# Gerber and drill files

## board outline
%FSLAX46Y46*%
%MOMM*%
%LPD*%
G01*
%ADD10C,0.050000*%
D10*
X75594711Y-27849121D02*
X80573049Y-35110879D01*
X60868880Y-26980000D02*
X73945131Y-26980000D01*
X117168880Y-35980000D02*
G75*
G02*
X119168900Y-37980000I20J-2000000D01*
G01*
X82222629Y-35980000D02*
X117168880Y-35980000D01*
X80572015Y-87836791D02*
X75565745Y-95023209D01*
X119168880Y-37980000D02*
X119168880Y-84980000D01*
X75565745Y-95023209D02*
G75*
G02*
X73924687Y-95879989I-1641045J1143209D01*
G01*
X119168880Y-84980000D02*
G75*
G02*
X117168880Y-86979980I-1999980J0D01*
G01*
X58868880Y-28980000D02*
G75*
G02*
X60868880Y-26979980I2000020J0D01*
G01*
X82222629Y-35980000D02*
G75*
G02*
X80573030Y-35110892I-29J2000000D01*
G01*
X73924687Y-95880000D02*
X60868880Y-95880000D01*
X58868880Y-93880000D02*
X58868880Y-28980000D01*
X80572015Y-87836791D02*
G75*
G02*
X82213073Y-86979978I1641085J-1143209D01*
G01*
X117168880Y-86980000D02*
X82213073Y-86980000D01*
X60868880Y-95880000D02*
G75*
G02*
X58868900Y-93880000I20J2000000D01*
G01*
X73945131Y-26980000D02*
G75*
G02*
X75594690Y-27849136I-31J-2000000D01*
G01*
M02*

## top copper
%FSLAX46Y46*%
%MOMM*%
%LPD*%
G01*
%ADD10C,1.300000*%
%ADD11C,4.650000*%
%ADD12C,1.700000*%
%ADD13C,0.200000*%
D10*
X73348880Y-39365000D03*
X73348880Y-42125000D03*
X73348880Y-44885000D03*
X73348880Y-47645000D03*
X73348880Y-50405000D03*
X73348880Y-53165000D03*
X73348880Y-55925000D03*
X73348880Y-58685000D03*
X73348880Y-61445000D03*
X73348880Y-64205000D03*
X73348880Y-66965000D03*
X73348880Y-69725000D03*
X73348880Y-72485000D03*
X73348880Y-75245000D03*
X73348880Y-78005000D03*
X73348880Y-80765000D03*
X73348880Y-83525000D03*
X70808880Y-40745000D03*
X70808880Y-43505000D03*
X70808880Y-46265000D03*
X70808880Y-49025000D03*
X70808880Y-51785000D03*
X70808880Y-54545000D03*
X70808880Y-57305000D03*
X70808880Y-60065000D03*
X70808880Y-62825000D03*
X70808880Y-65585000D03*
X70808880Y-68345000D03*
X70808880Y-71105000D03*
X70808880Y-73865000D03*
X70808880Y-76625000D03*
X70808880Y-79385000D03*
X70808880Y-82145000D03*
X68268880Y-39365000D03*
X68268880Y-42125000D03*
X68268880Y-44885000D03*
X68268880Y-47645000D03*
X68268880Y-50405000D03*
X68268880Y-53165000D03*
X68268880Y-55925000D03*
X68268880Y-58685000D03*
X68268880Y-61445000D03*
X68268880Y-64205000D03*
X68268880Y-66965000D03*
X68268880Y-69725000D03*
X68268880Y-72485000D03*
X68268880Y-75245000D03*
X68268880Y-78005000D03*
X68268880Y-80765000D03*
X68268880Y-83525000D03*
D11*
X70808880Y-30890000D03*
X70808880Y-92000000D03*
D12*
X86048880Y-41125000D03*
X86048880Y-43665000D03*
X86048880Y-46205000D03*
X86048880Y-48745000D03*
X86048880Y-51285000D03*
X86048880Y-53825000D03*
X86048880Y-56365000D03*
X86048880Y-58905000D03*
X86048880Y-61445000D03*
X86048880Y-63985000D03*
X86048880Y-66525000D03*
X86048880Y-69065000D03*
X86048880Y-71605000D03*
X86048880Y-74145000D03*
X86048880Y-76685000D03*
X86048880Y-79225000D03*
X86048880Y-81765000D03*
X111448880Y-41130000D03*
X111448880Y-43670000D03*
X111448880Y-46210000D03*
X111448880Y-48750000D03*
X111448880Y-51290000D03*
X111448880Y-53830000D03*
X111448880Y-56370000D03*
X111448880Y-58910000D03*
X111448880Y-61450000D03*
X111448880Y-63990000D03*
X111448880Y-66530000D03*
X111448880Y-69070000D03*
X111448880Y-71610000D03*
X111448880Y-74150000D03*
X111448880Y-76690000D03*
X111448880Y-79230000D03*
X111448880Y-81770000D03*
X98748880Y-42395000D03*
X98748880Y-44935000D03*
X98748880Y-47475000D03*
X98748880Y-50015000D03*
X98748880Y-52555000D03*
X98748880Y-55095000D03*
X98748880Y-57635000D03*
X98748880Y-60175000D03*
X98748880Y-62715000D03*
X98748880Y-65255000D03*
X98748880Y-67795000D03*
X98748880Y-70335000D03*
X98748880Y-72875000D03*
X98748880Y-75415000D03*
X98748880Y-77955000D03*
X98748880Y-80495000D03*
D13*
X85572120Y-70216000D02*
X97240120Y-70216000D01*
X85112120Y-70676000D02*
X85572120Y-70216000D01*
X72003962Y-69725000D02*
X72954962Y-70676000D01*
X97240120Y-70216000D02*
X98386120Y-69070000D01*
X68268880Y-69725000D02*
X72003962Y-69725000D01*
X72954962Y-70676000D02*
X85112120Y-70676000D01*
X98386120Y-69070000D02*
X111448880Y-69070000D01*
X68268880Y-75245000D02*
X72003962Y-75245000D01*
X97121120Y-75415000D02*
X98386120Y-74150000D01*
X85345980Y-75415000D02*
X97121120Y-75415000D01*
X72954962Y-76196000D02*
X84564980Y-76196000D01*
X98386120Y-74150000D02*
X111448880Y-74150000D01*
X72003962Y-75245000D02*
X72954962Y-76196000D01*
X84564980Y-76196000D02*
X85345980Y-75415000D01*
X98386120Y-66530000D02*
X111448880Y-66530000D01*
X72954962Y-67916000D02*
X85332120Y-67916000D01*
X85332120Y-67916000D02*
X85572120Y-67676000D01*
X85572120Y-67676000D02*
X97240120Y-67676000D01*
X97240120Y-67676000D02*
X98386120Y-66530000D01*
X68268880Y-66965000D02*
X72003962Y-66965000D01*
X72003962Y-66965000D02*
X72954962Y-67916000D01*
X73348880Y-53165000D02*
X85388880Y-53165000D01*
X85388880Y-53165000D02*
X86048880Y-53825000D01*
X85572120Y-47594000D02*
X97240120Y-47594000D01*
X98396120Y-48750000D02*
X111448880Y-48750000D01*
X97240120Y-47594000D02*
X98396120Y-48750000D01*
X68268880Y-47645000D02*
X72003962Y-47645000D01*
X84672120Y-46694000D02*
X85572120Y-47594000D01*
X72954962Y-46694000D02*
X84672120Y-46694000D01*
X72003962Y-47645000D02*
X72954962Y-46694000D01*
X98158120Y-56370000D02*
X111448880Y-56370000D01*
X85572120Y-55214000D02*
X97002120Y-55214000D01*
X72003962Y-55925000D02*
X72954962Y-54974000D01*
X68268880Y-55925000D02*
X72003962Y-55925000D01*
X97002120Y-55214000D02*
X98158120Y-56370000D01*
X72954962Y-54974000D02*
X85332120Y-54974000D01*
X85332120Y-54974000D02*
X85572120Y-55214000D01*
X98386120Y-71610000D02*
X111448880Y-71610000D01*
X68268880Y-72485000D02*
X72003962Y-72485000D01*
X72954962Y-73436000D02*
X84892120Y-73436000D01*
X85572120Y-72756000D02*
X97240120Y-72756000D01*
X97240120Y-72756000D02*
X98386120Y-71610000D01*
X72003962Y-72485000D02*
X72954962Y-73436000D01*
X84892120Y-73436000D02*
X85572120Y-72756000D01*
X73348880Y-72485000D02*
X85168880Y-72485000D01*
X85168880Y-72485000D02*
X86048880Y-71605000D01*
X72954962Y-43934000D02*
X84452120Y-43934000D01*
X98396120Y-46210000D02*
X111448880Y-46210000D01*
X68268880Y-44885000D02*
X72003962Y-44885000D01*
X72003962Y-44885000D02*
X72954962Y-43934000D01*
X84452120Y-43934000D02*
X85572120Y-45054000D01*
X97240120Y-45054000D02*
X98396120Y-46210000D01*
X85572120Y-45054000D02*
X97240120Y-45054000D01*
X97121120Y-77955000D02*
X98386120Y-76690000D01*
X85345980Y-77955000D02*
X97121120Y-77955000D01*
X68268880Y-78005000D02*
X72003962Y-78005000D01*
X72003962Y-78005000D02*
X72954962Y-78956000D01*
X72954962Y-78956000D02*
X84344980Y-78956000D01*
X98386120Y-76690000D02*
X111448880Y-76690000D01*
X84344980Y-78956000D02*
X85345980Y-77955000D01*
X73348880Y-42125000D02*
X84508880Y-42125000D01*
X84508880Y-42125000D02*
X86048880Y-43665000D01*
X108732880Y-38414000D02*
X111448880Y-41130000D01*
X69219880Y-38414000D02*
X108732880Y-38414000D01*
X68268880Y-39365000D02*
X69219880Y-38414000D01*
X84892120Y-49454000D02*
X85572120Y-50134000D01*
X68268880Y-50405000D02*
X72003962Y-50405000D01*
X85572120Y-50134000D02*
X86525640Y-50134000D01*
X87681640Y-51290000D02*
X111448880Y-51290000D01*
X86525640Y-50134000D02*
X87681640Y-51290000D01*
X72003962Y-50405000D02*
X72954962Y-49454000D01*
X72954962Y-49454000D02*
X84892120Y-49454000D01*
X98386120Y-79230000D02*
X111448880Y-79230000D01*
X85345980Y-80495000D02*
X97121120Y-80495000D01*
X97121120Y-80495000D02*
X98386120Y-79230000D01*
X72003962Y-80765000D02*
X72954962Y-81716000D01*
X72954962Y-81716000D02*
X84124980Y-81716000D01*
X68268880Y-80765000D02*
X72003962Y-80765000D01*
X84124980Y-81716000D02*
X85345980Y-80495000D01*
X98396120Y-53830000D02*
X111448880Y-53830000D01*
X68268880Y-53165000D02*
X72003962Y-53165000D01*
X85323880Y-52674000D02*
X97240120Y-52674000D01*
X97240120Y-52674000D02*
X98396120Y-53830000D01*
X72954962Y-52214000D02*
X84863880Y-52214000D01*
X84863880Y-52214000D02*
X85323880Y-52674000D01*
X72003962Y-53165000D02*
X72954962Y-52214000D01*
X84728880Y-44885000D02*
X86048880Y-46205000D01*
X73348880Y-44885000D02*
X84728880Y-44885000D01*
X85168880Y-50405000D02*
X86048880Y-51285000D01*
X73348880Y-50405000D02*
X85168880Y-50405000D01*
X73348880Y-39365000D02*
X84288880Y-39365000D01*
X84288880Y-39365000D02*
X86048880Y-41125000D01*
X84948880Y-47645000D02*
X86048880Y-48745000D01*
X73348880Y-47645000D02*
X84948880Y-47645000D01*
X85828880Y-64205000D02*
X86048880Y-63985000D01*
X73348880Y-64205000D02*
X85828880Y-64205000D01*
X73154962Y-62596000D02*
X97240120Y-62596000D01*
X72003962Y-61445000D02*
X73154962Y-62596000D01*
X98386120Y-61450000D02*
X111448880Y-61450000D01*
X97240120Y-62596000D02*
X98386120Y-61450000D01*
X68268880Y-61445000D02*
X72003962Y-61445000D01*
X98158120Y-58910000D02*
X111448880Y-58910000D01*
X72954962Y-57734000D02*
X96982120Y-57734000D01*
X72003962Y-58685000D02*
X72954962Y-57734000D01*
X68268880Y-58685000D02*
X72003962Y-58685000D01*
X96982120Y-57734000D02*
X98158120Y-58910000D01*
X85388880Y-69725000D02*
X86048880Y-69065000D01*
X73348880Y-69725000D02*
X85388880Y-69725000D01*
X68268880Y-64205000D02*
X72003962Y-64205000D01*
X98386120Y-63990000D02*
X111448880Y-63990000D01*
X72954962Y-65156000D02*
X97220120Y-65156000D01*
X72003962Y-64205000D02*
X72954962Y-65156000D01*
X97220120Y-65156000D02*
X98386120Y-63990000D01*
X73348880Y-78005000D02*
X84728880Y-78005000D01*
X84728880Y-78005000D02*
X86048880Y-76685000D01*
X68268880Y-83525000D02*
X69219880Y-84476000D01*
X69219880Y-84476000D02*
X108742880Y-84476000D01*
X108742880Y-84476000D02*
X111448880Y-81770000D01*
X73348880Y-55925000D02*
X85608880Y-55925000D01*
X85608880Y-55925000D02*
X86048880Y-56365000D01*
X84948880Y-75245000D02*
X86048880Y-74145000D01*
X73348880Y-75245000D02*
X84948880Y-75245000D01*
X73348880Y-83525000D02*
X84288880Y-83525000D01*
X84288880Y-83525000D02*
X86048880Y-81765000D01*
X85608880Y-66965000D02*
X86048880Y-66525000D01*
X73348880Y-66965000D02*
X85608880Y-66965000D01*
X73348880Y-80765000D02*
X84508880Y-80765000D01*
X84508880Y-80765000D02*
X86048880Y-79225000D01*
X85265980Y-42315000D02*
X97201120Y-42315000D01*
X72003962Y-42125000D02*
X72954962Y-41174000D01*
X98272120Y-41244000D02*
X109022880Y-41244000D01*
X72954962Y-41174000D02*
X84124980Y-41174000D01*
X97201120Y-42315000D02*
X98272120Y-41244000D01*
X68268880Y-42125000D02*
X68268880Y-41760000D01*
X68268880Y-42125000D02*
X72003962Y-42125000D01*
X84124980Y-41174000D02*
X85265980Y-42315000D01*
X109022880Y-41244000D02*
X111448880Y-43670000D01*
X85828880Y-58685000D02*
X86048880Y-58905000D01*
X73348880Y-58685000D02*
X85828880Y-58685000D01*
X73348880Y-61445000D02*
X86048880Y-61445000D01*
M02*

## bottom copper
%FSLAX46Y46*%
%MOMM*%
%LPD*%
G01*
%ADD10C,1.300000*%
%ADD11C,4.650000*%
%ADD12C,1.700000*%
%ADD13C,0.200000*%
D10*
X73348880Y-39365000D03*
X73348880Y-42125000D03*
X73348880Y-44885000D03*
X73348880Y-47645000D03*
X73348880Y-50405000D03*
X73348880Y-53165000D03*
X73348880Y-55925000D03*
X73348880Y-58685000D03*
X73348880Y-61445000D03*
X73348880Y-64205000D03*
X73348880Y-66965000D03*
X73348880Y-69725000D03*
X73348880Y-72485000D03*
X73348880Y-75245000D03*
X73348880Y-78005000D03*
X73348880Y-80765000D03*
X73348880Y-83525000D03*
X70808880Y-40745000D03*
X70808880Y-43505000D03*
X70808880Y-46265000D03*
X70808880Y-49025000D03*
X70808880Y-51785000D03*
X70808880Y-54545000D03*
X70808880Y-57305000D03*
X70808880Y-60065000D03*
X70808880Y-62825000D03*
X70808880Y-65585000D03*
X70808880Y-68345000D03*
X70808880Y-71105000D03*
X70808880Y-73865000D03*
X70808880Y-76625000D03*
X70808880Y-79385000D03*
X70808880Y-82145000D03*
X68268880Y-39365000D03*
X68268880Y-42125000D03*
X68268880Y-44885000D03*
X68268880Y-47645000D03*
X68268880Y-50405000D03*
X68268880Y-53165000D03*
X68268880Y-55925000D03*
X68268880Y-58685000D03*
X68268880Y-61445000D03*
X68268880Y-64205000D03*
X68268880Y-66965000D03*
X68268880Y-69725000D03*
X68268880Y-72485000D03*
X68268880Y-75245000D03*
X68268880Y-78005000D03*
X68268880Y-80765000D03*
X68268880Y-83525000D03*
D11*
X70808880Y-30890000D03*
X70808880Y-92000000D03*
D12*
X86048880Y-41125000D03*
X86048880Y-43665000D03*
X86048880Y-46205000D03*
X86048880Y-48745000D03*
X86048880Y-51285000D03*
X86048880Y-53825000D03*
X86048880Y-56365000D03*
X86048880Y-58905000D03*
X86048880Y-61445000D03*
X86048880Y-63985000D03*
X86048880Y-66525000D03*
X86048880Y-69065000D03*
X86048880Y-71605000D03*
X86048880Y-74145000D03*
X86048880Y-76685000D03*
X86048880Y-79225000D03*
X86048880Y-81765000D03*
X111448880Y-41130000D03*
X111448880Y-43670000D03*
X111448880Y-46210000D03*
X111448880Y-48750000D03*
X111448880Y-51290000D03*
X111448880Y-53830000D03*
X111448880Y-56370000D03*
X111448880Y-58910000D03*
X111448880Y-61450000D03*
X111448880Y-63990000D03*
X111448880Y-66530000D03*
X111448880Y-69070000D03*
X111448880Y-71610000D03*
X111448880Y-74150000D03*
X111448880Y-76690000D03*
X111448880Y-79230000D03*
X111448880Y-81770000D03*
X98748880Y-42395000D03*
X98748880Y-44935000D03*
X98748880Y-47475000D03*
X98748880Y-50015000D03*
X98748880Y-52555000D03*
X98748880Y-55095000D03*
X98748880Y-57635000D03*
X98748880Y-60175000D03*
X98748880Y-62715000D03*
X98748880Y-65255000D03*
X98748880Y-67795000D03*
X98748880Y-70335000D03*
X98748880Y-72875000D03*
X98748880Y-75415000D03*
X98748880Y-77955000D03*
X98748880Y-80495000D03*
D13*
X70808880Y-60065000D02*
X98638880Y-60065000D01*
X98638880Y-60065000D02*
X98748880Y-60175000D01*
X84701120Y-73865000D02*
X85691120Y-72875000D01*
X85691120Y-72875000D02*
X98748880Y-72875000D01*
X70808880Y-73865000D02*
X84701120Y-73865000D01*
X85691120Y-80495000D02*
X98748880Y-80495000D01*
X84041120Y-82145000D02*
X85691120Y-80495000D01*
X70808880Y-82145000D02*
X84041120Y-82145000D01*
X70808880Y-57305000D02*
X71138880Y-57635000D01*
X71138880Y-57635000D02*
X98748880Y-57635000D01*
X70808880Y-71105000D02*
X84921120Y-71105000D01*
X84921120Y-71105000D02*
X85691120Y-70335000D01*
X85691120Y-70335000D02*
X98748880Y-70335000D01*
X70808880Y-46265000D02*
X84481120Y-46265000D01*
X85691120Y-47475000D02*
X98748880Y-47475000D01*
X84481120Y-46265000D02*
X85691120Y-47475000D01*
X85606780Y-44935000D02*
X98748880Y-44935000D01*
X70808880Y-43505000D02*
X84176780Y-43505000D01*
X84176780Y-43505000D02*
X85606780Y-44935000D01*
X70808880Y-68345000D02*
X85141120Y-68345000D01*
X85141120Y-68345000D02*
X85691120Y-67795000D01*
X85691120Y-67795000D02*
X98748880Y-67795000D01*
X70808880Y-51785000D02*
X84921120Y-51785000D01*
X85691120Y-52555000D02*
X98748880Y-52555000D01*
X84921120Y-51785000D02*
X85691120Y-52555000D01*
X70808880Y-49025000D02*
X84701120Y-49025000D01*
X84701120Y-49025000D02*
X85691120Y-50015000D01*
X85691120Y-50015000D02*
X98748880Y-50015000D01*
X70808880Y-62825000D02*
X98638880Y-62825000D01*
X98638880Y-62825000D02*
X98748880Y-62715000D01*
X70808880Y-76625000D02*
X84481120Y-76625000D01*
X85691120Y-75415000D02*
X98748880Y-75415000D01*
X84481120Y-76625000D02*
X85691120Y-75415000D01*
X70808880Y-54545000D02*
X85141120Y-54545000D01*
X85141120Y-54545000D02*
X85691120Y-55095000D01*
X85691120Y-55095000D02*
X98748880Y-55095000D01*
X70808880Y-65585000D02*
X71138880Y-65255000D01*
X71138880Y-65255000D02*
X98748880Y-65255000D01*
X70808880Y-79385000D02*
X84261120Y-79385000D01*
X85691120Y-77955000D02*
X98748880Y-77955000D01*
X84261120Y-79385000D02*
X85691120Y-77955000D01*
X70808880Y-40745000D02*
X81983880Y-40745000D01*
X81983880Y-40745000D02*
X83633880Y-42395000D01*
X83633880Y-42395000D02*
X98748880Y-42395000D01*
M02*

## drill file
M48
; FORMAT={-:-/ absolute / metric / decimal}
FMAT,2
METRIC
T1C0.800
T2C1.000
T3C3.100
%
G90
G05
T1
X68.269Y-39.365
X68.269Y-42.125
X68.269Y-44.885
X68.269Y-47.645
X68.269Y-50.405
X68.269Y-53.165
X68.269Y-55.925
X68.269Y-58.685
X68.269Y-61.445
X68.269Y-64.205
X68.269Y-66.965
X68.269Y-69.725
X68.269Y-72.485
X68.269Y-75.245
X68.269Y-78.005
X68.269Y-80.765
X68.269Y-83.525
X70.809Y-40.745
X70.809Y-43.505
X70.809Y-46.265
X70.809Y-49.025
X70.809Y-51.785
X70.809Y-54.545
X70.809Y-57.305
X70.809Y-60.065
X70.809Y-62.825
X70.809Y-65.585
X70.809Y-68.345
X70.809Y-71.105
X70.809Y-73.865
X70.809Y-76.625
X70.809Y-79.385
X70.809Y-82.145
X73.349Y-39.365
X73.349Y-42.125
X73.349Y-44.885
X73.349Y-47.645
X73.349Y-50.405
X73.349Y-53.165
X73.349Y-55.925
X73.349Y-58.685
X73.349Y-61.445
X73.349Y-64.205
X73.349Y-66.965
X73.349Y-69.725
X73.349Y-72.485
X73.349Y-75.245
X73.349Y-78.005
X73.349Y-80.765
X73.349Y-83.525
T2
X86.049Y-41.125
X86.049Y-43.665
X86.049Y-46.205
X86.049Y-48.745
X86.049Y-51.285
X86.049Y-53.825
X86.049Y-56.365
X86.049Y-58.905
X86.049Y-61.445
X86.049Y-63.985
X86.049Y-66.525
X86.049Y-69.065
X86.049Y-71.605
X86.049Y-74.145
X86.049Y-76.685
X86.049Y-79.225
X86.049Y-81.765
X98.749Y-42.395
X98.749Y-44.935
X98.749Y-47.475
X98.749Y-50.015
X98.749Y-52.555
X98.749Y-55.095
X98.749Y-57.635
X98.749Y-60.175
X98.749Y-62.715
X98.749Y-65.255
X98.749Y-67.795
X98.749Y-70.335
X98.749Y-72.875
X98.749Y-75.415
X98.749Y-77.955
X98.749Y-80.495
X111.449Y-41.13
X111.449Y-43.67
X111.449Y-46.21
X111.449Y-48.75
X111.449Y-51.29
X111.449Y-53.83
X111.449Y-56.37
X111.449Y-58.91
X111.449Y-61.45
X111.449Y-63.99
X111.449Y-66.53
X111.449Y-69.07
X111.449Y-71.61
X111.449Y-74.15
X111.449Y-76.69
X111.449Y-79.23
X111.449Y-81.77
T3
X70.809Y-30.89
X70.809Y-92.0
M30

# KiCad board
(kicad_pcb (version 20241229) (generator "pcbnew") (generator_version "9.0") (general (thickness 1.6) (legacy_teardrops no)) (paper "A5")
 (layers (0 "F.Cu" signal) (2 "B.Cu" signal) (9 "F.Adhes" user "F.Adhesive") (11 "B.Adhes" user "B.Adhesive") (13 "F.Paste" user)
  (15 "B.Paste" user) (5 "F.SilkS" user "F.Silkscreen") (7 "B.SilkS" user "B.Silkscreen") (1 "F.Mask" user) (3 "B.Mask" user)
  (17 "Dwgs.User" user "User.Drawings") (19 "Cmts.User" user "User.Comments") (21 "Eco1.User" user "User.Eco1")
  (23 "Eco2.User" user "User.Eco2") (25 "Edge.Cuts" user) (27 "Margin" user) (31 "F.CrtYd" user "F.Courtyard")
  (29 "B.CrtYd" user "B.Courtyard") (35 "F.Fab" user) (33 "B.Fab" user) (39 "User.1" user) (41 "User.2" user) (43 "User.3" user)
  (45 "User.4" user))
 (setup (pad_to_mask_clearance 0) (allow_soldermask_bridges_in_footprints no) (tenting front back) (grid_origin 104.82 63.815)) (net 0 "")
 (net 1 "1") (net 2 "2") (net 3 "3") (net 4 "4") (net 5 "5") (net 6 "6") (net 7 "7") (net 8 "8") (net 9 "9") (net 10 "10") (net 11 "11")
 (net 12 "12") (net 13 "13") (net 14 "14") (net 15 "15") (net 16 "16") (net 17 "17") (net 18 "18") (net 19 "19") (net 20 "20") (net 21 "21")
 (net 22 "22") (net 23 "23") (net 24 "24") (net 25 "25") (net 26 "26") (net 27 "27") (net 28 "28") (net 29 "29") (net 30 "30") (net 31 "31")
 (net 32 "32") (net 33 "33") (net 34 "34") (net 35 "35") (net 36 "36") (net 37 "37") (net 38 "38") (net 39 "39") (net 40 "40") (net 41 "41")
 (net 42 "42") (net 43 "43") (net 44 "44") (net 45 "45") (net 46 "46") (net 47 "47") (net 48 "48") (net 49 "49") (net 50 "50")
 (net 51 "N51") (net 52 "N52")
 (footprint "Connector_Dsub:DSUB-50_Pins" (layer "F.Cu") (at 73.34888 39.365 -90)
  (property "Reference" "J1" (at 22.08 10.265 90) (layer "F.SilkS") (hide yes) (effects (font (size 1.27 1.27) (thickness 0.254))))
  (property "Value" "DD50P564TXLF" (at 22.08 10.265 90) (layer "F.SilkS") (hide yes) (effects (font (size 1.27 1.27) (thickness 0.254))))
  (pad "1" thru_hole circle (at 0 0 270) (size 1.3 1.3) (drill 0.8) (layers "*.Cu" "*.Mask") (remove_unused_layers no) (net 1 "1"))
  (pad "2" thru_hole circle (at 2.76 0 270) (size 1.3 1.3) (drill 0.8) (layers "*.Cu" "*.Mask") (remove_unused_layers no) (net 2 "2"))
  (pad "3" thru_hole circle (at 5.52 0 270) (size 1.3 1.3) (drill 0.8) (layers "*.Cu" "*.Mask") (remove_unused_layers no) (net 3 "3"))
  (pad "4" thru_hole circle (at 8.28 0 270) (size 1.3 1.3) (drill 0.8) (layers "*.Cu" "*.Mask") (remove_unused_layers no) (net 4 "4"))
  (pad "5" thru_hole circle (at 11.04 0 270) (size 1.3 1.3) (drill 0.8) (layers "*.Cu" "*.Mask") (remove_unused_layers no) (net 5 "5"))
  (pad "6" thru_hole circle (at 13.8 0 270) (size 1.3 1.3) (drill 0.8) (layers "*.Cu" "*.Mask") (remove_unused_layers no) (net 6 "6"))
  (pad "7" thru_hole circle (at 16.56 0 270) (size 1.3 1.3) (drill 0.8) (layers "*.Cu" "*.Mask") (remove_unused_layers no) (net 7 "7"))
  (pad "8" thru_hole circle (at 19.32 0 270) (size 1.3 1.3) (drill 0.8) (layers "*.Cu" "*.Mask") (remove_unused_layers no) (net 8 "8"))
  (pad "9" thru_hole circle (at 22.08 0 270) (size 1.3 1.3) (drill 0.8) (layers "*.Cu" "*.Mask") (remove_unused_layers no) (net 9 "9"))
  (pad "10" thru_hole circle (at 24.84 0 270) (size 1.3 1.3) (drill 0.8) (layers "*.Cu" "*.Mask") (remove_unused_layers no) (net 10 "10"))
  (pad "11" thru_hole circle (at 27.6 0 270) (size 1.3 1.3) (drill 0.8) (layers "*.Cu" "*.Mask") (remove_unused_layers no) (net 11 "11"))
  (pad "12" thru_hole circle (at 30.36 0 270) (size 1.3 1.3) (drill 0.8) (layers "*.Cu" "*.Mask") (remove_unused_layers no) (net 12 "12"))
  (pad "13" thru_hole circle (at 33.12 0 270) (size 1.3 1.3) (drill 0.8) (layers "*.Cu" "*.Mask") (remove_unused_layers no) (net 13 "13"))
  (pad "14" thru_hole circle (at 35.88 0 270) (size 1.3 1.3) (drill 0.8) (layers "*.Cu" "*.Mask") (remove_unused_layers no) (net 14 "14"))
  (pad "15" thru_hole circle (at 38.64 0 270) (size 1.3 1.3) (drill 0.8) (layers "*.Cu" "*.Mask") (remove_unused_layers no) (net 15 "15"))
  (pad "16" thru_hole circle (at 41.4 0 270) (size 1.3 1.3) (drill 0.8) (layers "*.Cu" "*.Mask") (remove_unused_layers no) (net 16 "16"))
  (pad "17" thru_hole circle (at 44.16 0 270) (size 1.3 1.3) (drill 0.8) (layers "*.Cu" "*.Mask") (remove_unused_layers no) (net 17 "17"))
  (pad "18" thru_hole circle (at 1.38 2.54 270) (size 1.3 1.3) (drill 0.8) (layers "*.Cu" "*.Mask") (remove_unused_layers no) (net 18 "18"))
  (pad "19" thru_hole circle (at 4.14 2.54 270) (size 1.3 1.3) (drill 0.8) (layers "*.Cu" "*.Mask") (remove_unused_layers no) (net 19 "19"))
  (pad "20" thru_hole circle (at 6.9 2.54 270) (size 1.3 1.3) (drill 0.8) (layers "*.Cu" "*.Mask") (remove_unused_layers no) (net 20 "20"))
  (pad "21" thru_hole circle (at 9.66 2.54 270) (size 1.3 1.3) (drill 0.8) (layers "*.Cu" "*.Mask") (remove_unused_layers no) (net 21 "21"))
  (pad "22" thru_hole circle (at 12.42 2.54 270) (size 1.3 1.3) (drill 0.8) (layers "*.Cu" "*.Mask") (remove_unused_layers no) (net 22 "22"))
  (pad "23" thru_hole circle (at 15.18 2.54 270) (size 1.3 1.3) (drill 0.8) (layers "*.Cu" "*.Mask") (remove_unused_layers no) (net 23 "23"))
  (pad "24" thru_hole circle (at 17.94 2.54 270) (size 1.3 1.3) (drill 0.8) (layers "*.Cu" "*.Mask") (remove_unused_layers no) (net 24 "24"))
  (pad "25" thru_hole circle (at 20.7 2.54 270) (size 1.3 1.3) (drill 0.8) (layers "*.Cu" "*.Mask") (remove_unused_layers no) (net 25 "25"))
  (pad "26" thru_hole circle (at 23.46 2.54 270) (size 1.3 1.3) (drill 0.8) (layers "*.Cu" "*.Mask") (remove_unused_layers no) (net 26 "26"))
  (pad "27" thru_hole circle (at 26.22 2.54 270) (size 1.3 1.3) (drill 0.8) (layers "*.Cu" "*.Mask") (remove_unused_layers no) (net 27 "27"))
  (pad "28" thru_hole circle (at 28.98 2.54 270) (size 1.3 1.3) (drill 0.8) (layers "*.Cu" "*.Mask") (remove_unused_layers no) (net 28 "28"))
  (pad "29" thru_hole circle (at 31.74 2.54 270) (size 1.3 1.3) (drill 0.8) (layers "*.Cu" "*.Mask") (remove_unused_layers no) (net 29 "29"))
  (pad "30" thru_hole circle (at 34.5 2.54 270) (size 1.3 1.3) (drill 0.8) (layers "*.Cu" "*.Mask") (remove_unused_layers no) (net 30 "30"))
  (pad "31" thru_hole circle (at 37.26 2.54 270) (size 1.3 1.3) (drill 0.8) (layers "*.Cu" "*.Mask") (remove_unused_layers no) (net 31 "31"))
  (pad "32" thru_hole circle (at 40.02 2.54 270) (size 1.3 1.3) (drill 0.8) (layers "*.Cu" "*.Mask") (remove_unused_layers no) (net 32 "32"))
  (pad "33" thru_hole circle (at 42.78 2.54 270) (size 1.3 1.3) (drill 0.8) (layers "*.Cu" "*.Mask") (remove_unused_layers no) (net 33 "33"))
  (pad "34" thru_hole circle (at 0 5.08 270) (size 1.3 1.3) (drill 0.8) (layers "*.Cu" "*.Mask") (remove_unused_layers no) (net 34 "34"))
  (pad "35" thru_hole circle (at 2.76 5.08 270) (size 1.3 1.3) (drill 0.8) (layers "*.Cu" "*.Mask") (remove_unused_layers no) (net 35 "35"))
  (pad "36" thru_hole circle (at 5.52 5.08 270) (size 1.3 1.3) (drill 0.8) (layers "*.Cu" "*.Mask") (remove_unused_layers no) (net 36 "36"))
  (pad "37" thru_hole circle (at 8.28 5.08 270) (size 1.3 1.3) (drill 0.8) (layers "*.Cu" "*.Mask") (remove_unused_layers no) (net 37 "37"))
  (pad "38" thru_hole circle (at 11.04 5.08 270) (size 1.3 1.3) (drill 0.8) (layers "*.Cu" "*.Mask") (remove_unused_layers no) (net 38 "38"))
  (pad "39" thru_hole circle (at 13.8 5.08 270) (size 1.3 1.3) (drill 0.8) (layers "*.Cu" "*.Mask") (remove_unused_layers no) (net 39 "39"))
  (pad "40" thru_hole circle (at 16.56 5.08 270) (size 1.3 1.3) (drill 0.8) (layers "*.Cu" "*.Mask") (remove_unused_layers no) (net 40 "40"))
  (pad "41" thru_hole circle (at 19.32 5.08 270) (size 1.3 1.3) (drill 0.8) (layers "*.Cu" "*.Mask") (remove_unused_layers no) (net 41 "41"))
  (pad "42" thru_hole circle (at 22.08 5.08 270) (size 1.3 1.3) (drill 0.8) (layers "*.Cu" "*.Mask") (remove_unused_layers no) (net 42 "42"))
  (pad "43" thru_hole circle (at 24.84 5.08 270) (size 1.3 1.3) (drill 0.8) (layers "*.Cu" "*.Mask") (remove_unused_layers no) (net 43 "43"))
  (pad "44" thru_hole circle (at 27.6 5.08 270) (size 1.3 1.3) (drill 0.8) (layers "*.Cu" "*.Mask") (remove_unused_layers no) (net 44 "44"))
  (pad "45" thru_hole circle (at 30.36 5.08 270) (size 1.3 1.3) (drill 0.8) (layers "*.Cu" "*.Mask") (remove_unused_layers no) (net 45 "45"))
  (pad "46" thru_hole circle (at 33.12 5.08 270) (size 1.3 1.3) (drill 0.8) (layers "*.Cu" "*.Mask") (remove_unused_layers no) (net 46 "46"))
  (pad "47" thru_hole circle (at 35.88 5.08 270) (size 1.3 1.3) (drill 0.8) (layers "*.Cu" "*.Mask") (remove_unused_layers no) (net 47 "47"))
  (pad "48" thru_hole circle (at 38.64 5.08 270) (size 1.3 1.3) (drill 0.8) (layers "*.Cu" "*.Mask") (remove_unused_layers no) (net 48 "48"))
  (pad "49" thru_hole circle (at 41.4 5.08 270) (size 1.3 1.3) (drill 0.8) (layers "*.Cu" "*.Mask") (remove_unused_layers no) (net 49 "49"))
  (pad "50" thru_hole circle (at 44.16 5.08 270) (size 1.3 1.3) (drill 0.8) (layers "*.Cu" "*.Mask") (remove_unused_layers no) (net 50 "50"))
  (pad "MH1" thru_hole circle (at -8.475 2.54 270) (size 4.65 4.65) (drill 3.1) (layers "*.Cu" "*.Mask") (remove_unused_layers no)
   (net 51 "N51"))
  (pad "MH2" thru_hole circle (at 52.635 2.54 270) (size 4.65 4.65) (drill 3.1) (layers "*.Cu" "*.Mask") (remove_unused_layers no)
   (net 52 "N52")))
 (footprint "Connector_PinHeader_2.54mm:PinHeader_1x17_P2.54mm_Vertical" (layer "F.Cu") (at 86.04888 41.125)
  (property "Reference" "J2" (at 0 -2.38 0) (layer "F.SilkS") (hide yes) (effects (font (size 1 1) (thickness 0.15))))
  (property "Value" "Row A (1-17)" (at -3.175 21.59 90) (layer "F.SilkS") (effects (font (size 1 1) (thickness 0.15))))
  (pad "1" thru_hole circle (at 0 0) (size 1.7 1.7) (drill 1) (layers "*.Cu" "*.Mask") (remove_unused_layers no) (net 1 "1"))
  (pad "2" thru_hole circle (at 0 2.54) (size 1.7 1.7) (drill 1) (layers "*.Cu" "*.Mask") (remove_unused_layers no) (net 2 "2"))
  (pad "3" thru_hole circle (at 0 5.08) (size 1.7 1.7) (drill 1) (layers "*.Cu" "*.Mask") (remove_unused_layers no) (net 3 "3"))
  (pad "4" thru_hole circle (at 0 7.62) (size 1.7 1.7) (drill 1) (layers "*.Cu" "*.Mask") (remove_unused_layers no) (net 4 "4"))
  (pad "5" thru_hole circle (at 0 10.16) (size 1.7 1.7) (drill 1) (layers "*.Cu" "*.Mask") (remove_unused_layers no) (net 5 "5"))
  (pad "6" thru_hole circle (at 0 12.7) (size 1.7 1.7) (drill 1) (layers "*.Cu" "*.Mask") (remove_unused_layers no) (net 6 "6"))
  (pad "7" thru_hole circle (at 0 15.24) (size 1.7 1.7) (drill 1) (layers "*.Cu" "*.Mask") (remove_unused_layers no) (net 7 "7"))
  (pad "8" thru_hole circle (at 0 17.78) (size 1.7 1.7) (drill 1) (layers "*.Cu" "*.Mask") (remove_unused_layers no) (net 8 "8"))
  (pad "9" thru_hole circle (at 0 20.32) (size 1.7 1.7) (drill 1) (layers "*.Cu" "*.Mask") (remove_unused_layers no) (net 9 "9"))
  (pad "10" thru_hole circle (at 0 22.86) (size 1.7 1.7) (drill 1) (layers "*.Cu" "*.Mask") (remove_unused_layers no) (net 10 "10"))
  (pad "11" thru_hole circle (at 0 25.4) (size 1.7 1.7) (drill 1) (layers "*.Cu" "*.Mask") (remove_unused_layers no) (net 11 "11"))
  (pad "12" thru_hole circle (at 0 27.94) (size 1.7 1.7) (drill 1) (layers "*.Cu" "*.Mask") (remove_unused_layers no) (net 12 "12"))
  (pad "13" thru_hole circle (at 0 30.48) (size 1.7 1.7) (drill 1) (layers "*.Cu" "*.Mask") (remove_unused_layers no) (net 13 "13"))
  (pad "14" thru_hole circle (at 0 33.02) (size 1.7 1.7) (drill 1) (layers "*.Cu" "*.Mask") (remove_unused_layers no) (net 14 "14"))
  (pad "15" thru_hole circle (at 0 35.56) (size 1.7 1.7) (drill 1) (layers "*.Cu" "*.Mask") (remove_unused_layers no) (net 15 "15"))
  (pad "16" thru_hole circle (at 0 38.1) (size 1.7 1.7) (drill 1) (layers "*.Cu" "*.Mask") (remove_unused_layers no) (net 16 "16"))
  (pad "17" thru_hole circle (at 0 40.64) (size 1.7 1.7) (drill 1) (layers "*.Cu" "*.Mask") (remove_unused_layers no) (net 17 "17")))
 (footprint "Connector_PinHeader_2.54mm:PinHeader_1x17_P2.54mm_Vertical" (layer "F.Cu") (at 111.44888 41.13)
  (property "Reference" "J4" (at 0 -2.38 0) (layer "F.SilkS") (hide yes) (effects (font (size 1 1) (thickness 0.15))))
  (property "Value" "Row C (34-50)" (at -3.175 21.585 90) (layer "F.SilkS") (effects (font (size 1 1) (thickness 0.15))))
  (pad "1" thru_hole circle (at 0 0) (size 1.7 1.7) (drill 1) (layers "*.Cu" "*.Mask") (remove_unused_layers no) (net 34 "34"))
  (pad "2" thru_hole circle (at 0 2.54) (size 1.7 1.7) (drill 1) (layers "*.Cu" "*.Mask") (remove_unused_layers no) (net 35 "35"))
  (pad "3" thru_hole circle (at 0 5.08) (size 1.7 1.7) (drill 1) (layers "*.Cu" "*.Mask") (remove_unused_layers no) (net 36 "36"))
  (pad "4" thru_hole circle (at 0 7.62) (size 1.7 1.7) (drill 1) (layers "*.Cu" "*.Mask") (remove_unused_layers no) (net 37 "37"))
  (pad "5" thru_hole circle (at 0 10.16) (size 1.7 1.7) (drill 1) (layers "*.Cu" "*.Mask") (remove_unused_layers no) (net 38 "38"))
  (pad "6" thru_hole circle (at 0 12.7) (size 1.7 1.7) (drill 1) (layers "*.Cu" "*.Mask") (remove_unused_layers no) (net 39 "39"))
  (pad "7" thru_hole circle (at 0 15.24) (size 1.7 1.7) (drill 1) (layers "*.Cu" "*.Mask") (remove_unused_layers no) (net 40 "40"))
  (pad "8" thru_hole circle (at 0 17.78) (size 1.7 1.7) (drill 1) (layers "*.Cu" "*.Mask") (remove_unused_layers no) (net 41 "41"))
  (pad "9" thru_hole circle (at 0 20.32) (size 1.7 1.7) (drill 1) (layers "*.Cu" "*.Mask") (remove_unused_layers no) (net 42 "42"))
  (pad "10" thru_hole circle (at 0 22.86) (size 1.7 1.7) (drill 1) (layers "*.Cu" "*.Mask") (remove_unused_layers no) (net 43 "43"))
  (pad "11" thru_hole circle (at 0 25.4) (size 1.7 1.7) (drill 1) (layers "*.Cu" "*.Mask") (remove_unused_layers no) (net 44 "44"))
  (pad "12" thru_hole circle (at 0 27.94) (size 1.7 1.7) (drill 1) (layers "*.Cu" "*.Mask") (remove_unused_layers no) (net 45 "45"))
  (pad "13" thru_hole circle (at 0 30.48) (size 1.7 1.7) (drill 1) (layers "*.Cu" "*.Mask") (remove_unused_layers no) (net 46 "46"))
  (pad "14" thru_hole circle (at 0 33.02) (size 1.7 1.7) (drill 1) (layers "*.Cu" "*.Mask") (remove_unused_layers no) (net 47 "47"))
  (pad "15" thru_hole circle (at 0 35.56) (size 1.7 1.7) (drill 1) (layers "*.Cu" "*.Mask") (remove_unused_layers no) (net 48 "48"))
  (pad "16" thru_hole circle (at 0 38.1) (size 1.7 1.7) (drill 1) (layers "*.Cu" "*.Mask") (remove_unused_layers no) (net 49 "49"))
  (pad "17" thru_hole circle (at 0 40.64) (size 1.7 1.7) (drill 1) (layers "*.Cu" "*.Mask") (remove_unused_layers no) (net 50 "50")))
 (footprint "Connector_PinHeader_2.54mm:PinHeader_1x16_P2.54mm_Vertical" (layer "F.Cu") (at 98.74888 42.395)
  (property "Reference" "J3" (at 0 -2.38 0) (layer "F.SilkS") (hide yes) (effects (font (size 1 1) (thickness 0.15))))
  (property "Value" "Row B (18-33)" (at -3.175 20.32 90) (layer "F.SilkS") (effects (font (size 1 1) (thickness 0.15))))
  (pad "1" thru_hole circle (at 0 0) (size 1.7 1.7) (drill 1) (layers "*.Cu" "*.Mask") (remove_unused_layers no) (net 18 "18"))
  (pad "2" thru_hole circle (at 0 2.54) (size 1.7 1.7) (drill 1) (layers "*.Cu" "*.Mask") (remove_unused_layers no) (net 19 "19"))
  (pad "3" thru_hole circle (at 0 5.08) (size 1.7 1.7) (drill 1) (layers "*.Cu" "*.Mask") (remove_unused_layers no) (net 20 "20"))
  (pad "4" thru_hole circle (at 0 7.62) (size 1.7 1.7) (drill 1) (layers "*.Cu" "*.Mask") (remove_unused_layers no) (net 21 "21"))
  (pad "5" thru_hole circle (at 0 10.16) (size 1.7 1.7) (drill 1) (layers "*.Cu" "*.Mask") (remove_unused_layers no) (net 22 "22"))
  (pad "6" thru_hole circle (at 0 12.7) (size 1.7 1.7) (drill 1) (layers "*.Cu" "*.Mask") (remove_unused_layers no) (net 23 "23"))
  (pad "7" thru_hole circle (at 0 15.24) (size 1.7 1.7) (drill 1) (layers "*.Cu" "*.Mask") (remove_unused_layers no) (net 24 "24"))
  (pad "8" thru_hole circle (at 0 17.78) (size 1.7 1.7) (drill 1) (layers "*.Cu" "*.Mask") (remove_unused_layers no) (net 25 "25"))
  (pad "9" thru_hole circle (at 0 20.32) (size 1.7 1.7) (drill 1) (layers "*.Cu" "*.Mask") (remove_unused_layers no) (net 26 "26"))
  (pad "10" thru_hole circle (at 0 22.86) (size 1.7 1.7) (drill 1) (layers "*.Cu" "*.Mask") (remove_unused_layers no) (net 27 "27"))
  (pad "11" thru_hole circle (at 0 25.4) (size 1.7 1.7) (drill 1) (layers "*.Cu" "*.Mask") (remove_unused_layers no) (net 28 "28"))
  (pad "12" thru_hole circle (at 0 27.94) (size 1.7 1.7) (drill 1) (layers "*.Cu" "*.Mask") (remove_unused_layers no) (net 29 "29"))
  (pad "13" thru_hole circle (at 0 30.48) (size 1.7 1.7) (drill 1) (layers "*.Cu" "*.Mask") (remove_unused_layers no) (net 30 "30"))
  (pad "14" thru_hole circle (at 0 33.02) (size 1.7 1.7) (drill 1) (layers "*.Cu" "*.Mask") (remove_unused_layers no) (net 31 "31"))
  (pad "15" thru_hole circle (at 0 35.56) (size 1.7 1.7) (drill 1) (layers "*.Cu" "*.Mask") (remove_unused_layers no) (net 32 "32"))
  (pad "16" thru_hole circle (at 0 38.1) (size 1.7 1.7) (drill 1) (layers "*.Cu" "*.Mask") (remove_unused_layers no) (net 33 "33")))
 (gr_line (start 75.594711 27.849121) (end 80.573049 35.110879) (stroke (width 0.05) (type default)) (layer "Edge.Cuts"))
 (gr_line (start 60.86888 26.98) (end 73.945131 26.98) (stroke (width 0.05) (type default)) (layer "Edge.Cuts"))
 (gr_arc (start 117.16888 35.98) (mid 118.583094 36.565786) (end 119.16888 37.98) (stroke (width 0.05) (type default)) (layer "Edge.Cuts"))
 (gr_line (start 82.222629 35.98) (end 117.16888 35.98) (stroke (width 0.05) (type default)) (layer "Edge.Cuts"))
 (gr_line (start 80.572015 87.836791) (end 75.565745 95.023209) (stroke (width 0.05) (type default)) (layer "Edge.Cuts"))
 (gr_line (start 119.16888 37.98) (end 119.16888 84.98) (stroke (width 0.05) (type default)) (layer "Edge.Cuts"))
 (gr_arc (start 75.565745 95.023209) (mid 74.850317 95.652909) (end 73.924687 95.88) (stroke (width 0.05) (type default))
  (layer "Edge.Cuts"))
 (gr_arc (start 119.16888 84.98) (mid 118.583094 86.394214) (end 117.16888 86.98) (stroke (width 0.05) (type default)) (layer "Edge.Cuts"))
 (gr_arc (start 58.86888 28.98) (mid 59.454666 27.565786) (end 60.86888 26.98) (stroke (width 0.05) (type default)) (layer "Edge.Cuts"))
 (gr_arc (start 82.222629 35.98) (mid 81.290362 35.749429) (end 80.573049 35.110879) (stroke (width 0.05) (type default))
  (layer "Edge.Cuts"))
 (gr_line (start 73.924687 95.88) (end 60.86888 95.88) (stroke (width 0.05) (type default)) (layer "Edge.Cuts"))
 (gr_line (start 58.86888 93.88) (end 58.86888 28.98) (stroke (width 0.05) (type default)) (layer "Edge.Cuts"))
 (gr_arc (start 80.572015 87.836791) (mid 81.287443 87.207091) (end 82.213073 86.98) (stroke (width 0.05) (type default))
  (layer "Edge.Cuts"))
 (gr_line (start 117.16888 86.98) (end 82.213073 86.98) (stroke (width 0.05) (type default)) (layer "Edge.Cuts"))
 (gr_arc (start 60.86888 95.88) (mid 59.454666 95.294214) (end 58.86888 93.88) (stroke (width 0.05) (type default)) (layer "Edge.Cuts"))
 (gr_arc (start 73.945131 26.98) (mid 74.877398 27.210571) (end 75.594711 27.849121) (stroke (width 0.05) (type default))
  (layer "Edge.Cuts"))
 (segment (start 85.57212 70.216) (end 97.24012 70.216) (width 0.2) (layer "F.Cu") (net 45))
 (segment (start 85.11212 70.676) (end 85.57212 70.216) (width 0.2) (layer "F.Cu") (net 45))
 (segment (start 72.003962 69.725) (end 72.954962 70.676) (width 0.2) (layer "F.Cu") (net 45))
 (segment (start 97.24012 70.216) (end 98.38612 69.07) (width 0.2) (layer "F.Cu") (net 45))
 (segment (start 68.26888 69.725) (end 72.003962 69.725) (width 0.2) (layer "F.Cu") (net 45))
 (segment (start 72.954962 70.676) (end 85.11212 70.676) (width 0.2) (layer "F.Cu") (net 45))
 (segment (start 98.38612 69.07) (end 111.44888 69.07) (width 0.2) (layer "F.Cu") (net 45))
 (segment (start 68.26888 75.245) (end 72.003962 75.245) (width 0.2) (layer "F.Cu") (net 47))
 (segment (start 97.12112 75.415) (end 98.38612 74.15) (width 0.2) (layer "F.Cu") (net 47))
 (segment (start 85.34598 75.415) (end 97.12112 75.415) (width 0.2) (layer "F.Cu") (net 47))
 (segment (start 72.954962 76.196) (end 84.56498 76.196) (width 0.2) (layer "F.Cu") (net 47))
 (segment (start 98.38612 74.15) (end 111.44888 74.15) (width 0.2) (layer "F.Cu") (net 47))
 (segment (start 72.003962 75.245) (end 72.954962 76.196) (width 0.2) (layer "F.Cu") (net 47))
 (segment (start 84.56498 76.196) (end 85.34598 75.415) (width 0.2) (layer "F.Cu") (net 47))
 (segment (start 70.80888 60.065) (end 98.63888 60.065) (width 0.2) (layer "B.Cu") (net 25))
 (segment (start 98.63888 60.065) (end 98.74888 60.175) (width 0.2) (layer "B.Cu") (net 25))
 (segment (start 98.38612 66.53) (end 111.44888 66.53) (width 0.2) (layer "F.Cu") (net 44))
 (segment (start 72.954962 67.916) (end 85.33212 67.916) (width 0.2) (layer "F.Cu") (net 44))
 (segment (start 85.33212 67.916) (end 85.57212 67.676) (width 0.2) (layer "F.Cu") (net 44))
 (segment (start 85.57212 67.676) (end 97.24012 67.676) (width 0.2) (layer "F.Cu") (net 44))
 (segment (start 97.24012 67.676) (end 98.38612 66.53) (width 0.2) (layer "F.Cu") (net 44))
 (segment (start 68.26888 66.965) (end 72.003962 66.965) (width 0.2) (layer "F.Cu") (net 44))
 (segment (start 72.003962 66.965) (end 72.954962 67.916) (width 0.2) (layer "F.Cu") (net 44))
 (segment (start 73.34888 53.165) (end 85.38888 53.165) (width 0.2) (layer "F.Cu") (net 6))
 (segment (start 85.38888 53.165) (end 86.04888 53.825) (width 0.2) (layer "F.Cu") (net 6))
 (segment (start 85.57212 47.594) (end 97.24012 47.594) (width 0.2) (layer "F.Cu") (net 37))
 (segment (start 98.39612 48.75) (end 111.44888 48.75) (width 0.2) (layer "F.Cu") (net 37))
 (segment (start 97.24012 47.594) (end 98.39612 48.75) (width 0.2) (layer "F.Cu") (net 37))
 (segment (start 68.26888 47.645) (end 72.003962 47.645) (width 0.2) (layer "F.Cu") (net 37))
 (segment (start 84.67212 46.694) (end 85.57212 47.594) (width 0.2) (layer "F.Cu") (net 37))
 (segment (start 72.954962 46.694) (end 84.67212 46.694) (width 0.2) (layer "F.Cu") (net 37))
 (segment (start 72.003962 47.645) (end 72.954962 46.694) (width 0.2) (layer "F.Cu") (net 37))
 (segment (start 84.70112 73.865) (end 85.69112 72.875) (width 0.2) (layer "B.Cu") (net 30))
 (segment (start 85.69112 72.875) (end 98.74888 72.875) (width 0.2) (layer "B.Cu") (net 30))
 (segment (start 70.80888 73.865) (end 84.70112 73.865) (width 0.2) (layer "B.Cu") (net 30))
 (segment (start 85.69112 80.495) (end 98.74888 80.495) (width 0.2) (layer "B.Cu") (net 33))
 (segment (start 84.04112 82.145) (end 85.69112 80.495) (width 0.2) (layer "B.Cu") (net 33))
 (segment (start 70.80888 82.145) (end 84.04112 82.145) (width 0.2) (layer "B.Cu") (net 33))
 (segment (start 70.80888 57.305) (end 71.13888 57.635) (width 0.2) (layer "B.Cu") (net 24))
 (segment (start 71.13888 57.635) (end 98.74888 57.635) (width 0.2) (layer "B.Cu") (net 24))
 (segment (start 98.15812 56.37) (end 111.44888 56.37) (width 0.2) (layer "F.Cu") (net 40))
 (segment (start 85.57212 55.214) (end 97.00212 55.214) (width 0.2) (layer "F.Cu") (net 40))
 (segment (start 72.003962 55.925) (end 72.954962 54.974) (width 0.2) (layer "F.Cu") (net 40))
 (segment (start 68.26888 55.925) (end 72.003962 55.925) (width 0.2) (layer "F.Cu") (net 40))
 (segment (start 97.00212 55.214) (end 98.15812 56.37) (width 0.2) (layer "F.Cu") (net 40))
 (segment (start 72.954962 54.974) (end 85.33212 54.974) (width 0.2) (layer "F.Cu") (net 40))
 (segment (start 85.33212 54.974) (end 85.57212 55.214) (width 0.2) (layer "F.Cu") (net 40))
 (segment (start 98.38612 71.61) (end 111.44888 71.61) (width 0.2) (layer "F.Cu") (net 46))
 (segment (start 68.26888 72.485) (end 72.003962 72.485) (width 0.2) (layer "F.Cu") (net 46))
 (segment (start 72.954962 73.436) (end 84.89212 73.436) (width 0.2) (layer "F.Cu") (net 46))
 (segment (start 85.57212 72.756) (end 97.24012 72.756) (width 0.2) (layer "F.Cu") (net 46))
 (segment (start 97.24012 72.756) (end 98.38612 71.61) (width 0.2) (layer "F.Cu") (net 46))
 (segment (start 72.003962 72.485) (end 72.954962 73.436) (width 0.2) (layer "F.Cu") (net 46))
 (segment (start 84.89212 73.436) (end 85.57212 72.756) (width 0.2) (layer "F.Cu") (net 46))
 (segment (start 73.34888 72.485) (end 85.16888 72.485) (width 0.2) (layer "F.Cu") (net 13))
 (segment (start 85.16888 72.485) (end 86.04888 71.605) (width 0.2) (layer "F.Cu") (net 13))
 (segment (start 72.954962 43.934) (end 84.45212 43.934) (width 0.2) (layer "F.Cu") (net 36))
 (segment (start 98.39612 46.21) (end 111.44888 46.21) (width 0.2) (layer "F.Cu") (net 36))
 (segment (start 68.26888 44.885) (end 72.003962 44.885) (width 0.2) (layer "F.Cu") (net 36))
 (segment (start 72.003962 44.885) (end 72.954962 43.934) (width 0.2) (layer "F.Cu") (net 36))
 (segment (start 84.45212 43.934) (end 85.57212 45.054) (width 0.2) (layer "F.Cu") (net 36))
 (segment (start 97.24012 45.054) (end 98.39612 46.21) (width 0.2) (layer "F.Cu") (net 36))
 (segment (start 85.57212 45.054) (end 97.24012 45.054) (width 0.2) (layer "F.Cu") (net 36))
 (segment (start 97.12112 77.955) (end 98.38612 76.69) (width 0.2) (layer "F.Cu") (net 48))
 (segment (start 85.34598 77.955) (end 97.12112 77.955) (width 0.2) (layer "F.Cu") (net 48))
 (segment (start 68.26888 78.005) (end 72.003962 78.005) (width 0.2) (layer "F.Cu") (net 48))
 (segment (start 72.003962 78.005) (end 72.954962 78.956) (width 0.2) (layer "F.Cu") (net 48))
 (segment (start 72.954962 78.956) (end 84.34498 78.956) (width 0.2) (layer "F.Cu") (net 48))
 (segment (start 98.38612 76.69) (end 111.44888 76.69) (width 0.2) (layer "F.Cu") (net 48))
 (segment (start 84.34498 78.956) (end 85.34598 77.955) (width 0.2) (layer "F.Cu") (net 48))
 (segment (start 73.34888 42.125) (end 84.50888 42.125) (width 0.2) (layer "F.Cu") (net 2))
 (segment (start 84.50888 42.125) (end 86.04888 43.665) (width 0.2) (layer "F.Cu") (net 2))
 (segment (start 70.80888 71.105) (end 84.92112 71.105) (width 0.2) (layer "B.Cu") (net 29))
 (segment (start 84.92112 71.105) (end 85.69112 70.335) (width 0.2) (layer "B.Cu") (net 29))
 (segment (start 85.69112 70.335) (end 98.74888 70.335) (width 0.2) (layer "B.Cu") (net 29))
 (segment (start 108.73288 38.414) (end 111.44888 41.13) (width 0.2) (layer "F.Cu") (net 34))
 (segment (start 69.21988 38.414) (end 108.73288 38.414) (width 0.2) (layer "F.Cu") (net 34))
 (segment (start 68.26888 39.365) (end 69.21988 38.414) (width 0.2) (layer "F.Cu") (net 34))
 (segment (start 84.89212 49.454) (end 85.57212 50.134) (width 0.2) (layer "F.Cu") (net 38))
 (segment (start 68.26888 50.405) (end 72.003962 50.405) (width 0.2) (layer "F.Cu") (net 38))
 (segment (start 85.57212 50.134) (end 86.52564 50.134) (width 0.2) (layer "F.Cu") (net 38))
 (segment (start 87.68164 51.29) (end 111.44888 51.29) (width 0.2) (layer "F.Cu") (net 38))
 (segment (start 86.52564 50.134) (end 87.68164 51.29) (width 0.2) (layer "F.Cu") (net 38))
 (segment (start 72.003962 50.405) (end 72.954962 49.454) (width 0.2) (layer "F.Cu") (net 38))
 (segment (start 72.954962 49.454) (end 84.89212 49.454) (width 0.2) (layer "F.Cu") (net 38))
 (segment (start 70.80888 46.265) (end 84.48112 46.265) (width 0.2) (layer "B.Cu") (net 20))
 (segment (start 85.69112 47.475) (end 98.74888 47.475) (width 0.2) (layer "B.Cu") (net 20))
 (segment (start 84.48112 46.265) (end 85.69112 47.475) (width 0.2) (layer "B.Cu") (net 20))
 (segment (start 98.38612 79.23) (end 111.44888 79.23) (width 0.2) (layer "F.Cu") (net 49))
 (segment (start 85.34598 80.495) (end 97.12112 80.495) (width 0.2) (layer "F.Cu") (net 49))
 (segment (start 97.12112 80.495) (end 98.38612 79.23) (width 0.2) (layer "F.Cu") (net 49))
 (segment (start 72.003962 80.765) (end 72.954962 81.716) (width 0.2) (layer "F.Cu") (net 49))
 (segment (start 72.954962 81.716) (end 84.12498 81.716) (width 0.2) (layer "F.Cu") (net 49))
 (segment (start 68.26888 80.765) (end 72.003962 80.765) (width 0.2) (layer "F.Cu") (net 49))
 (segment (start 84.12498 81.716) (end 85.34598 80.495) (width 0.2) (layer "F.Cu") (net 49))
 (segment (start 98.39612 53.83) (end 111.44888 53.83) (width 0.2) (layer "F.Cu") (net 39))
 (segment (start 68.26888 53.165) (end 72.003962 53.165) (width 0.2) (layer "F.Cu") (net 39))
 (segment (start 85.32388 52.674) (end 97.24012 52.674) (width 0.2) (layer "F.Cu") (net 39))
 (segment (start 97.24012 52.674) (end 98.39612 53.83) (width 0.2) (layer "F.Cu") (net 39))
 (segment (start 72.954962 52.214) (end 84.86388 52.214) (width 0.2) (layer "F.Cu") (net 39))
 (segment (start 84.86388 52.214) (end 85.32388 52.674) (width 0.2) (layer "F.Cu") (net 39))
 (segment (start 72.003962 53.165) (end 72.954962 52.214) (width 0.2) (layer "F.Cu") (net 39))
 (segment (start 84.72888 44.885) (end 86.04888 46.205) (width 0.2) (layer "F.Cu") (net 3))
 (segment (start 73.34888 44.885) (end 84.72888 44.885) (width 0.2) (layer "F.Cu") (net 3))
 (segment (start 85.16888 50.405) (end 86.04888 51.285) (width 0.2) (layer "F.Cu") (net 5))
 (segment (start 73.34888 50.405) (end 85.16888 50.405) (width 0.2) (layer "F.Cu") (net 5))
 (segment (start 85.60678 44.935) (end 98.74888 44.935) (width 0.2) (layer "B.Cu") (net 19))
 (segment (start 70.80888 43.505) (end 84.17678 43.505) (width 0.2) (layer "B.Cu") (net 19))
 (segment (start 84.17678 43.505) (end 85.60678 44.935) (width 0.2) (layer "B.Cu") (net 19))
 (segment (start 73.34888 39.365) (end 84.28888 39.365) (width 0.2) (layer "F.Cu") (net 1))
 (segment (start 84.28888 39.365) (end 86.04888 41.125) (width 0.2) (layer "F.Cu") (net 1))
 (segment (start 84.94888 47.645) (end 86.04888 48.745) (width 0.2) (layer "F.Cu") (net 4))
 (segment (start 73.34888 47.645) (end 84.94888 47.645) (width 0.2) (layer "F.Cu") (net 4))
 (segment (start 85.82888 64.205) (end 86.04888 63.985) (width 0.2) (layer "F.Cu") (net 10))
 (segment (start 73.34888 64.205) (end 85.82888 64.205) (width 0.2) (layer "F.Cu") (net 10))
 (segment (start 70.80888 68.345) (end 85.14112 68.345) (width 0.2) (layer "B.Cu") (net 28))
 (segment (start 85.14112 68.345) (end 85.69112 67.795) (width 0.2) (layer "B.Cu") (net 28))
 (segment (start 85.69112 67.795) (end 98.74888 67.795) (width 0.2) (layer "B.Cu") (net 28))
 (segment (start 70.80888 51.785) (end 84.92112 51.785) (width 0.2) (layer "B.Cu") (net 22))
 (segment (start 85.69112 52.555) (end 98.74888 52.555) (width 0.2) (layer "B.Cu") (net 22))
 (segment (start 84.92112 51.785) (end 85.69112 52.555) (width 0.2) (layer "B.Cu") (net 22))
 (segment (start 73.154962 62.596) (end 97.24012 62.596) (width 0.2) (layer "F.Cu") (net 42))
 (segment (start 72.003962 61.445) (end 73.154962 62.596) (width 0.2) (layer "F.Cu") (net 42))
 (segment (start 98.38612 61.45) (end 111.44888 61.45) (width 0.2) (layer "F.Cu") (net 42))
 (segment (start 97.24012 62.596) (end 98.38612 61.45) (width 0.2) (layer "F.Cu") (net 42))
 (segment (start 68.26888 61.445) (end 72.003962 61.445) (width 0.2) (layer "F.Cu") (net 42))
 (segment (start 70.80888 49.025) (end 84.70112 49.025) (width 0.2) (layer "B.Cu") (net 21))
 (segment (start 84.70112 49.025) (end 85.69112 50.015) (width 0.2) (layer "B.Cu") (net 21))
 (segment (start 85.69112 50.015) (end 98.74888 50.015) (width 0.2) (layer "B.Cu") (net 21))
 (segment (start 98.15812 58.91) (end 111.44888 58.91) (width 0.2) (layer "F.Cu") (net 41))
 (segment (start 72.954962 57.734) (end 96.98212 57.734) (width 0.2) (layer "F.Cu") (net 41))
 (segment (start 72.003962 58.685) (end 72.954962 57.734) (width 0.2) (layer "F.Cu") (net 41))
 (segment (start 68.26888 58.685) (end 72.003962 58.685) (width 0.2) (layer "F.Cu") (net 41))
 (segment (start 96.98212 57.734) (end 98.15812 58.91) (width 0.2) (layer "F.Cu") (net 41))
 (segment (start 85.38888 69.725) (end 86.04888 69.065) (width 0.2) (layer "F.Cu") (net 12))
 (segment (start 73.34888 69.725) (end 85.38888 69.725) (width 0.2) (layer "F.Cu") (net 12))
 (segment (start 68.26888 64.205) (end 72.003962 64.205) (width 0.2) (layer "F.Cu") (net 43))
 (segment (start 98.38612 63.99) (end 111.44888 63.99) (width 0.2) (layer "F.Cu") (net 43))
 (segment (start 72.954962 65.156) (end 97.22012 65.156) (width 0.2) (layer "F.Cu") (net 43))
 (segment (start 72.003962 64.205) (end 72.954962 65.156) (width 0.2) (layer "F.Cu") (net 43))
 (segment (start 97.22012 65.156) (end 98.38612 63.99) (width 0.2) (layer "F.Cu") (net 43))
 (segment (start 70.80888 62.825) (end 98.63888 62.825) (width 0.2) (layer "B.Cu") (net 26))
 (segment (start 98.63888 62.825) (end 98.74888 62.715) (width 0.2) (layer "B.Cu") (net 26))
 (segment (start 73.34888 78.005) (end 84.72888 78.005) (width 0.2) (layer "F.Cu") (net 15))
 (segment (start 84.72888 78.005) (end 86.04888 76.685) (width 0.2) (layer "F.Cu") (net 15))
 (segment (start 70.80888 76.625) (end 84.48112 76.625) (width 0.2) (layer "B.Cu") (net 31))
 (segment (start 85.69112 75.415) (end 98.74888 75.415) (width 0.2) (layer "B.Cu") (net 31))
 (segment (start 84.48112 76.625) (end 85.69112 75.415) (width 0.2) (layer "B.Cu") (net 31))
 (segment (start 68.26888 83.525) (end 69.21988 84.476) (width 0.2) (layer "F.Cu") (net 50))
 (segment (start 69.21988 84.476) (end 108.74288 84.476) (width 0.2) (layer "F.Cu") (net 50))
 (segment (start 108.74288 84.476) (end 111.44888 81.77) (width 0.2) (layer "F.Cu") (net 50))
 (segment (start 73.34888 55.925) (end 85.60888 55.925) (width 0.2) (layer "F.Cu") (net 7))
 (segment (start 85.60888 55.925) (end 86.04888 56.365) (width 0.2) (layer "F.Cu") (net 7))
 (segment (start 70.80888 54.545) (end 85.14112 54.545) (width 0.2) (layer "B.Cu") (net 23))
 (segment (start 85.14112 54.545) (end 85.69112 55.095) (width 0.2) (layer "B.Cu") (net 23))
 (segment (start 85.69112 55.095) (end 98.74888 55.095) (width 0.2) (layer "B.Cu") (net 23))
 (segment (start 84.94888 75.245) (end 86.04888 74.145) (width 0.2) (layer "F.Cu") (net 14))
 (segment (start 73.34888 75.245) (end 84.94888 75.245) (width 0.2) (layer "F.Cu") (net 14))
 (segment (start 73.34888 83.525) (end 84.28888 83.525) (width 0.2) (layer "F.Cu") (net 17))
 (segment (start 84.28888 83.525) (end 86.04888 81.765) (width 0.2) (layer "F.Cu") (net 17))
 (segment (start 85.60888 66.965) (end 86.04888 66.525) (width 0.2) (layer "F.Cu") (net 11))
 (segment (start 73.34888 66.965) (end 85.60888 66.965) (width 0.2) (layer "F.Cu") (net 11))
 (segment (start 70.80888 65.585) (end 71.13888 65.255) (width 0.2) (layer "B.Cu") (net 27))
 (segment (start 71.13888 65.255) (end 98.74888 65.255) (width 0.2) (layer "B.Cu") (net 27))
 (segment (start 73.34888 80.765) (end 84.50888 80.765) (width 0.2) (layer "F.Cu") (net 16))
 (segment (start 84.50888 80.765) (end 86.04888 79.225) (width 0.2) (layer "F.Cu") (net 16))
 (segment (start 70.80888 79.385) (end 84.26112 79.385) (width 0.2) (layer "B.Cu") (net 32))
 (segment (start 85.69112 77.955) (end 98.74888 77.955) (width 0.2) (layer "B.Cu") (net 32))
 (segment (start 84.26112 79.385) (end 85.69112 77.955) (width 0.2) (layer "B.Cu") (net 32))
 (segment (start 85.26598 42.315) (end 97.20112 42.315) (width 0.2) (layer "F.Cu") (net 35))
 (segment (start 72.003962 42.125) (end 72.954962 41.174) (width 0.2) (layer "F.Cu") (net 35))
 (segment (start 98.27212 41.244) (end 109.02288 41.244) (width 0.2) (layer "F.Cu") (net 35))
 (segment (start 72.954962 41.174) (end 84.12498 41.174) (width 0.2) (layer "F.Cu") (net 35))
 (segment (start 97.20112 42.315) (end 98.27212 41.244) (width 0.2) (layer "F.Cu") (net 35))
 (segment (start 68.26888 42.125) (end 68.26888 41.76) (width 0.2) (layer "F.Cu") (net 35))
 (segment (start 68.26888 42.125) (end 72.003962 42.125) (width 0.2) (layer "F.Cu") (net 35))
 (segment (start 84.12498 41.174) (end 85.26598 42.315) (width 0.2) (layer "F.Cu") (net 35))
 (segment (start 109.02288 41.244) (end 111.44888 43.67) (width 0.2) (layer "F.Cu") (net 35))
 (segment (start 85.82888 58.685) (end 86.04888 58.905) (width 0.2) (layer "F.Cu") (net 8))
 (segment (start 73.34888 58.685) (end 85.82888 58.685) (width 0.2) (layer "F.Cu") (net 8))
 (segment (start 70.80888 40.745) (end 81.98388 40.745) (width 0.2) (layer "B.Cu") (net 18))
 (segment (start 81.98388 40.745) (end 83.63388 42.395) (width 0.2) (layer "B.Cu") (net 18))
 (segment (start 83.63388 42.395) (end 98.74888 42.395) (width 0.2) (layer "B.Cu") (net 18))
 (segment (start 73.34888 61.445) (end 86.04888 61.445) (width 0.2) (layer "F.Cu") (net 9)))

